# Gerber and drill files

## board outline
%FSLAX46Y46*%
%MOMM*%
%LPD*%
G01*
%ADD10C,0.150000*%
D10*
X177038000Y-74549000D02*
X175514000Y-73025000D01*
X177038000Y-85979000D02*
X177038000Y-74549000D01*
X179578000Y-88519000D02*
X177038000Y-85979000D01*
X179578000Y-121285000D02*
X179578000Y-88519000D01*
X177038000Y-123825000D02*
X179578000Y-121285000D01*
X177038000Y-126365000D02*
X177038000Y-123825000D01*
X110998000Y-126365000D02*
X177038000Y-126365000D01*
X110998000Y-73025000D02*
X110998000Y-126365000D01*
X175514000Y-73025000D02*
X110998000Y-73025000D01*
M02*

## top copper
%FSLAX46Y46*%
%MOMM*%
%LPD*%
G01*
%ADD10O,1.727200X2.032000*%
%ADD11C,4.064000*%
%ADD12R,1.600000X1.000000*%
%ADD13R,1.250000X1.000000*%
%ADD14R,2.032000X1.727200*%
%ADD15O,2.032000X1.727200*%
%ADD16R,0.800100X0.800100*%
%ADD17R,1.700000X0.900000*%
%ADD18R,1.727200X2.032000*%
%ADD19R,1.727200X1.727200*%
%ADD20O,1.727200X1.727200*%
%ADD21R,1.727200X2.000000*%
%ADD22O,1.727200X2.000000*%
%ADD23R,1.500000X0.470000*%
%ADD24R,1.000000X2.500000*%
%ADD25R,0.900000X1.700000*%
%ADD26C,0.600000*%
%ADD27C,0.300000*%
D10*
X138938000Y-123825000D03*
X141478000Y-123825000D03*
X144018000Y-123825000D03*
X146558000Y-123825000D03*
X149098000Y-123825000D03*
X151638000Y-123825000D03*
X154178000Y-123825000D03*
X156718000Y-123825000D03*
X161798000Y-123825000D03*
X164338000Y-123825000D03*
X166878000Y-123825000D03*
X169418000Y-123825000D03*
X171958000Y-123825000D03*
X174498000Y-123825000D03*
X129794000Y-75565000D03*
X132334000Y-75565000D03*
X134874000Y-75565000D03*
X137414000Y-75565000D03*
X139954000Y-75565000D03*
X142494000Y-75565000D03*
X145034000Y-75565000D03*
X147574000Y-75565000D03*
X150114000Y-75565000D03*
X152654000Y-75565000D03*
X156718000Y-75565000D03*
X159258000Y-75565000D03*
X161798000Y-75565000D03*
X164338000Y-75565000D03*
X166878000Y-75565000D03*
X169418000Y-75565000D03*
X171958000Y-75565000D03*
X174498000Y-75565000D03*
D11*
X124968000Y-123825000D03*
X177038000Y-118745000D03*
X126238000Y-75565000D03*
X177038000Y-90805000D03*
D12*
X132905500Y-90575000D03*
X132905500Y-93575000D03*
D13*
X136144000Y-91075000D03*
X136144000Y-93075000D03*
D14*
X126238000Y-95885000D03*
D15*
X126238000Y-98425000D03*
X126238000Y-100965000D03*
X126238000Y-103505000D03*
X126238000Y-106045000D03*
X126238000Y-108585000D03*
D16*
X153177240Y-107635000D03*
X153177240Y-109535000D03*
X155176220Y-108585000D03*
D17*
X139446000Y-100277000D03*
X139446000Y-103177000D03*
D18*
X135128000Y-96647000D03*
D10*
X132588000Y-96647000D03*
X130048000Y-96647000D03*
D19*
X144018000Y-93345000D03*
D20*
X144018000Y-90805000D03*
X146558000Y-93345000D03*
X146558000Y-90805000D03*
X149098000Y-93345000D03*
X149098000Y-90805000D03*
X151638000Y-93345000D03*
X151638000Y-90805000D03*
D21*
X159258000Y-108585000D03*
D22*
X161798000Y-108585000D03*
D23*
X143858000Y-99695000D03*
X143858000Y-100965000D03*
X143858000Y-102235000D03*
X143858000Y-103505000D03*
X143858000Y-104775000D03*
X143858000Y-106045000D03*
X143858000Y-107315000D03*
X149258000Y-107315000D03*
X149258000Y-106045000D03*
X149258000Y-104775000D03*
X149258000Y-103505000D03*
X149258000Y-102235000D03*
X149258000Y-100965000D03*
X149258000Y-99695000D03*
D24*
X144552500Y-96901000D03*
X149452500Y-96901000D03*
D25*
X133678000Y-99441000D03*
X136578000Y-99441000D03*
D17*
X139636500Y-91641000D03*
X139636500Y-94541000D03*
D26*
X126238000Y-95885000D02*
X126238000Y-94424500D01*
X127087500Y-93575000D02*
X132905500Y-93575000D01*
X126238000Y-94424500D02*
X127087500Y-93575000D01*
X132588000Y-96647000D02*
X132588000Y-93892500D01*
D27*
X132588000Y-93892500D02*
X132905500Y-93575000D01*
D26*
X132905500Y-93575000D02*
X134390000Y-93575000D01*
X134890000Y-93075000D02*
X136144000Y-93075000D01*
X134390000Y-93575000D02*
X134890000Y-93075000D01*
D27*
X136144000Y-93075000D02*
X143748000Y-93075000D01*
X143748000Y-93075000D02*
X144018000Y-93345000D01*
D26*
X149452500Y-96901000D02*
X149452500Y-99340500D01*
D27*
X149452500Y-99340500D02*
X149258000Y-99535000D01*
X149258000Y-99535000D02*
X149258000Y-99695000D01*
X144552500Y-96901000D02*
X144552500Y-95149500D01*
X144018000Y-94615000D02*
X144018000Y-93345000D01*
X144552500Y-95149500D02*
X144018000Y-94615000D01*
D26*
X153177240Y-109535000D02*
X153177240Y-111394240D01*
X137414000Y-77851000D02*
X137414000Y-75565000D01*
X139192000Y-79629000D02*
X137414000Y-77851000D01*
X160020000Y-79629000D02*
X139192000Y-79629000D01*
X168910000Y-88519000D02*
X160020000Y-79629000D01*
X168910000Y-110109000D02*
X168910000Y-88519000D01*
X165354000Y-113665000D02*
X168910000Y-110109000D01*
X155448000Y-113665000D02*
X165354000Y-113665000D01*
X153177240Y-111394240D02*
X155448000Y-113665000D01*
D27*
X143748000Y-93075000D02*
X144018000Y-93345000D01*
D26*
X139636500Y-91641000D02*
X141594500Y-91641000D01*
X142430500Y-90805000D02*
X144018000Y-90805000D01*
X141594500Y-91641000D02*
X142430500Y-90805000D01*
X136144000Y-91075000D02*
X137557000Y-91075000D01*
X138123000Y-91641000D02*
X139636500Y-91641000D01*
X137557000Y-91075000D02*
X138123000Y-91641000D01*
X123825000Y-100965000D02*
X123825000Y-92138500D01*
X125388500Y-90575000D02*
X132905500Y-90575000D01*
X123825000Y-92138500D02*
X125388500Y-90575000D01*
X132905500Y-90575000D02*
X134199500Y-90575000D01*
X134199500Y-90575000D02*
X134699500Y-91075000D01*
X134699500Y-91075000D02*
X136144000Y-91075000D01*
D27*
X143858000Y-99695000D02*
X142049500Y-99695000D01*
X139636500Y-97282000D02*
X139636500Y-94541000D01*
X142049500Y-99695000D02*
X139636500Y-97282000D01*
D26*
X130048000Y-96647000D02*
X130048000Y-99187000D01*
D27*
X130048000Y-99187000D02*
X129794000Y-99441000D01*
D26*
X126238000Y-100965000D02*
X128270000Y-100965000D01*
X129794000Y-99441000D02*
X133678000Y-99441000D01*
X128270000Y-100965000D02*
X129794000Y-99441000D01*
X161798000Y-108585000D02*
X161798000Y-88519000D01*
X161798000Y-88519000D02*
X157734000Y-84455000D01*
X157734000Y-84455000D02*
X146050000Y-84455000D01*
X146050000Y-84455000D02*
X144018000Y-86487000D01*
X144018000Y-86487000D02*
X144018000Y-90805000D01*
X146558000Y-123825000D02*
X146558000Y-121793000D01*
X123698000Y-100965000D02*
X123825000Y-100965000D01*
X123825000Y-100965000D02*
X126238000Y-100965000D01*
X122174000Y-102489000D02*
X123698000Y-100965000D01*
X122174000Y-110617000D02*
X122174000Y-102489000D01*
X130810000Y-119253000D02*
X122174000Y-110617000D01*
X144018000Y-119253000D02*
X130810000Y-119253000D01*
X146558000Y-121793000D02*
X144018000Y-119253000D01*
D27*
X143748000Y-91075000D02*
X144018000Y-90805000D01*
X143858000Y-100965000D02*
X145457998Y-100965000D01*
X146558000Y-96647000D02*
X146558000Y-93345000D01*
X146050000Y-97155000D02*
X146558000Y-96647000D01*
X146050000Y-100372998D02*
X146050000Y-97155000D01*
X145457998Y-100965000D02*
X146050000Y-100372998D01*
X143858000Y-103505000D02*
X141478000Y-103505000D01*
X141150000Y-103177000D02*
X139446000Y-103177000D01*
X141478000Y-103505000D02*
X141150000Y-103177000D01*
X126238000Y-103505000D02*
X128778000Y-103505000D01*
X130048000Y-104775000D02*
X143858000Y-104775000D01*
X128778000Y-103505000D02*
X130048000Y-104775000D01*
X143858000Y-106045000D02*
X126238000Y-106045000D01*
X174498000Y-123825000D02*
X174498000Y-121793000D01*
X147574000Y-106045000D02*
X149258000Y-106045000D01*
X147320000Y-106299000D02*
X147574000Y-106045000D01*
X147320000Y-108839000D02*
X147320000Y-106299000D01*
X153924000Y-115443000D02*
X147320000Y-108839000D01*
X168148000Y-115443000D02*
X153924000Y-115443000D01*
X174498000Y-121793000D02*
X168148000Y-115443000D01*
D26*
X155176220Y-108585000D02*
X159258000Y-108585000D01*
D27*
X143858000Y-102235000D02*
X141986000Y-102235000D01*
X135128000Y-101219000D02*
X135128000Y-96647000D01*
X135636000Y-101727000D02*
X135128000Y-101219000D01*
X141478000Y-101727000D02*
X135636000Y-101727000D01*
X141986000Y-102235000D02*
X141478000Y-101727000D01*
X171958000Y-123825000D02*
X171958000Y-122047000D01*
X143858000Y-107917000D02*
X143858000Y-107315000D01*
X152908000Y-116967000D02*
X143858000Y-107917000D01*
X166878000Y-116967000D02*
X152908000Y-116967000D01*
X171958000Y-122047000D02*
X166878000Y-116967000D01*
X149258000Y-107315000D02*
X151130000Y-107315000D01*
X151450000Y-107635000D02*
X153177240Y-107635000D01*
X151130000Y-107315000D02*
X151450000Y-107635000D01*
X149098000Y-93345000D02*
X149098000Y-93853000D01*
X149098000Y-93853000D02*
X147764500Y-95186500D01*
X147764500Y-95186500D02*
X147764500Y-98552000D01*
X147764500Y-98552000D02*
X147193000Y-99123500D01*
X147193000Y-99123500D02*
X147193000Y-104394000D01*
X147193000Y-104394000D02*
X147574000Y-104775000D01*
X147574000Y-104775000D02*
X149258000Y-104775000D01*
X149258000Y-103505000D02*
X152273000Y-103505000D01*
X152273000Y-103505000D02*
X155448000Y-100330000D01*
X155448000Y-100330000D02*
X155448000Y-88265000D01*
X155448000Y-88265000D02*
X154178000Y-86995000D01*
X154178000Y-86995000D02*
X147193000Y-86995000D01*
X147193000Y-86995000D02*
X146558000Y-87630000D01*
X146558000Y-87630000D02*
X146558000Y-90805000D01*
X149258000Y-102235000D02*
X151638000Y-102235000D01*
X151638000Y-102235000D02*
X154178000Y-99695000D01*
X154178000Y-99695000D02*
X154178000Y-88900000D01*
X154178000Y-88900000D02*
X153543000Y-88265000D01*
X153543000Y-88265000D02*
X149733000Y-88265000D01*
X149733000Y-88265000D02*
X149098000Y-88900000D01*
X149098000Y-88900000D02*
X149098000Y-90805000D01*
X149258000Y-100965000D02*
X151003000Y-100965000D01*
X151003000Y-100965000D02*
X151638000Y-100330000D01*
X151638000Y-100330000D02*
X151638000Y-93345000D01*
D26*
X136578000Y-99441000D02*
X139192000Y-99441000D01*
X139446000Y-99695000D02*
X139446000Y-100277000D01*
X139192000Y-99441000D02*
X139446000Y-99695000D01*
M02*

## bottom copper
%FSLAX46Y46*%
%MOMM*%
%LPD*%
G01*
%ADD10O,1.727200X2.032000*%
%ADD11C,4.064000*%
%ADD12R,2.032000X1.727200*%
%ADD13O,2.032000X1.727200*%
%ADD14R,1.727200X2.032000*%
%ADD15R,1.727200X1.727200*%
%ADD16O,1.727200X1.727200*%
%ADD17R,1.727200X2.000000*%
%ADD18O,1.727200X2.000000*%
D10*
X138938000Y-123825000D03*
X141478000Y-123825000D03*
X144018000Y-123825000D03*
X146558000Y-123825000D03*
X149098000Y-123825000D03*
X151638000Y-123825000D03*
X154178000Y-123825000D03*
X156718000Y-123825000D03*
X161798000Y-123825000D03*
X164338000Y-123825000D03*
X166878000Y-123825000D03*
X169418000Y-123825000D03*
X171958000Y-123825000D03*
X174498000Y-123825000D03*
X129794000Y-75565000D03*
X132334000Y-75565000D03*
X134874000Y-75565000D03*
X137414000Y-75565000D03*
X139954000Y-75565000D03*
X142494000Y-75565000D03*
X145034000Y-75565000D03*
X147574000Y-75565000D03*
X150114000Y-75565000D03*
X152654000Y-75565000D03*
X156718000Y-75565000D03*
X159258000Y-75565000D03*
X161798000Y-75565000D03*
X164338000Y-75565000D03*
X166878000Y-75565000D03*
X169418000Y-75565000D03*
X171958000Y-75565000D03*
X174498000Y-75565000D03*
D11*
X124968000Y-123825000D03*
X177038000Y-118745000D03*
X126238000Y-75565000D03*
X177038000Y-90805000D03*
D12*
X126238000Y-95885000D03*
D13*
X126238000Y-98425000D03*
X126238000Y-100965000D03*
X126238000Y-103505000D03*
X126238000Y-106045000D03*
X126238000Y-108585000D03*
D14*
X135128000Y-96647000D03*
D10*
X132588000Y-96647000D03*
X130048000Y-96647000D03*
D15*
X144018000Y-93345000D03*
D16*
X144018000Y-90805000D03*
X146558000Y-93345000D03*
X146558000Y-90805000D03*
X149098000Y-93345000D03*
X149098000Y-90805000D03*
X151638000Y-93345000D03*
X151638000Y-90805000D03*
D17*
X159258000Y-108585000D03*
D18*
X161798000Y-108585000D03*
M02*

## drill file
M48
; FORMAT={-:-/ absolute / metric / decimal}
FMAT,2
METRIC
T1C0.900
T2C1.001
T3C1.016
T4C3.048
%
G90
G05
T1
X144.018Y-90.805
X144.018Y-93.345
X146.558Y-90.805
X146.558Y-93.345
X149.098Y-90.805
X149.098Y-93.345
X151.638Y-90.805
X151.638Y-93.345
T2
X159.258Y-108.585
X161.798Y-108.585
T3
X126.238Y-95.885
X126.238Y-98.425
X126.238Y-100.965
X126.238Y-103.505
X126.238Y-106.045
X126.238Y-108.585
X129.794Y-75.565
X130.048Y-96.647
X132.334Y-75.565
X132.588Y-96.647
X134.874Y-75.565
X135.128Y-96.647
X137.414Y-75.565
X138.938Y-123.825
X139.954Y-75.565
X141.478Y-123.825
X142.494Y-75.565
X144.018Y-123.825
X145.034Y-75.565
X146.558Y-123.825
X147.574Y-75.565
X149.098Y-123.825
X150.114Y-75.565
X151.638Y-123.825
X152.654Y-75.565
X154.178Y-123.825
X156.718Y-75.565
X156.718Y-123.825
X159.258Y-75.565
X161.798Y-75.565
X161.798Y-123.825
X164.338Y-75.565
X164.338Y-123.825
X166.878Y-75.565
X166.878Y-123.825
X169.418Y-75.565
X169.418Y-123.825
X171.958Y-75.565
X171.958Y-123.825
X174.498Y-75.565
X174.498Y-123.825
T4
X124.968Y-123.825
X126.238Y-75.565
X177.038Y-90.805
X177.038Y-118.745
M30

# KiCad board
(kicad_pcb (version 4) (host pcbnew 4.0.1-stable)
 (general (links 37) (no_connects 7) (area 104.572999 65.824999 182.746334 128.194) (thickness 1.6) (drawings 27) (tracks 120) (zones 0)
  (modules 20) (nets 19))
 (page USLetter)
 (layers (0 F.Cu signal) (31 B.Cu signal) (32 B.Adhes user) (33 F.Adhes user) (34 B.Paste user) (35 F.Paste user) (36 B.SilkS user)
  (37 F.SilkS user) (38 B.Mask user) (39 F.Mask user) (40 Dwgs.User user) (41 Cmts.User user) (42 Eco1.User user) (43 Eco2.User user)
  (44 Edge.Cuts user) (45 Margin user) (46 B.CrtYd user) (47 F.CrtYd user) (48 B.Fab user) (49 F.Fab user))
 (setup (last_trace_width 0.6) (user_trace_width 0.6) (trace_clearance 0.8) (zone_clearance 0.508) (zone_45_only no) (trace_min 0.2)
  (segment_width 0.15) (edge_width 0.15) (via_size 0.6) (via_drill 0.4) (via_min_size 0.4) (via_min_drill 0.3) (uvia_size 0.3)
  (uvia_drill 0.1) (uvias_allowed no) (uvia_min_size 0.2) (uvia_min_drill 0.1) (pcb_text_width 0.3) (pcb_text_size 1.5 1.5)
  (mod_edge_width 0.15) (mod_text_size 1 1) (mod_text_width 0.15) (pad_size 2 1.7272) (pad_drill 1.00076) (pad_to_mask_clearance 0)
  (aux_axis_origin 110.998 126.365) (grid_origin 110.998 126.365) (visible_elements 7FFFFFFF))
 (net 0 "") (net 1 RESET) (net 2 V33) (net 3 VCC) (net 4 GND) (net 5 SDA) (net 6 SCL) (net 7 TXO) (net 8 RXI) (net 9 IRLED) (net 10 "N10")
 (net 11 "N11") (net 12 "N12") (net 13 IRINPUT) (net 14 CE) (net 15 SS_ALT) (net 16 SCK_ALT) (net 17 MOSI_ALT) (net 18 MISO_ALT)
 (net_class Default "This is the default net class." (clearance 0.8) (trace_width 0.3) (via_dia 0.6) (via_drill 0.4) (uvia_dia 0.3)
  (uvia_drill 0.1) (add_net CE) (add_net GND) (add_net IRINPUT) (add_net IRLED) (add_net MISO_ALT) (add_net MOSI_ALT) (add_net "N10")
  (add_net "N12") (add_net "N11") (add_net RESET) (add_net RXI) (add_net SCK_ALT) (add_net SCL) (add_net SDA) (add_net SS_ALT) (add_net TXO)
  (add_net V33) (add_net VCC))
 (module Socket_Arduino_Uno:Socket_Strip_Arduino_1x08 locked (layer F.Cu) (at 138.938 123.825)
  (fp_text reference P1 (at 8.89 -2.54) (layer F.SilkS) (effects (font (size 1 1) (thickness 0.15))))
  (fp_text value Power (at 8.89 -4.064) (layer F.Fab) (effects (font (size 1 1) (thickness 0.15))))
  (pad 1 thru_hole oval (at 0 0) (size 1.7272 2.032) (drill 1.016) (layers *.Cu *.Mask F.SilkS))
  (pad 2 thru_hole oval (at 2.54 0) (size 1.7272 2.032) (drill 1.016) (layers *.Cu *.Mask F.SilkS))
  (pad 3 thru_hole oval (at 5.08 0) (size 1.7272 2.032) (drill 1.016) (layers *.Cu *.Mask F.SilkS) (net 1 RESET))
  (pad 4 thru_hole oval (at 7.62 0) (size 1.7272 2.032) (drill 1.016) (layers *.Cu *.Mask F.SilkS) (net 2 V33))
  (pad 5 thru_hole oval (at 10.16 0) (size 1.7272 2.032) (drill 1.016) (layers *.Cu *.Mask F.SilkS) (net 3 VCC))
  (pad 6 thru_hole oval (at 12.7 0) (size 1.7272 2.032) (drill 1.016) (layers *.Cu *.Mask F.SilkS) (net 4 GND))
  (pad 7 thru_hole oval (at 15.24 0) (size 1.7272 2.032) (drill 1.016) (layers *.Cu *.Mask F.SilkS) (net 4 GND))
  (pad 8 thru_hole oval (at 17.78 0) (size 1.7272 2.032) (drill 1.016) (layers *.Cu *.Mask F.SilkS)))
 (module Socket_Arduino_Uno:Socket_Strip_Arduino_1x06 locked (layer F.Cu) (at 161.798 123.825)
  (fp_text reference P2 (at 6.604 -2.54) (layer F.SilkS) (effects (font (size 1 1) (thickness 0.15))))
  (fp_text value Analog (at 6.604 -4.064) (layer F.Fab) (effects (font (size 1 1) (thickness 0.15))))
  (pad 1 thru_hole oval (at 0 0) (size 1.7272 2.032) (drill 1.016) (layers *.Cu *.Mask F.SilkS))
  (pad 2 thru_hole oval (at 2.54 0) (size 1.7272 2.032) (drill 1.016) (layers *.Cu *.Mask F.SilkS))
  (pad 3 thru_hole oval (at 5.08 0) (size 1.7272 2.032) (drill 1.016) (layers *.Cu *.Mask F.SilkS))
  (pad 4 thru_hole oval (at 7.62 0) (size 1.7272 2.032) (drill 1.016) (layers *.Cu *.Mask F.SilkS))
  (pad 5 thru_hole oval (at 10.16 0) (size 1.7272 2.032) (drill 1.016) (layers *.Cu *.Mask F.SilkS) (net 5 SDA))
  (pad 6 thru_hole oval (at 12.7 0) (size 1.7272 2.032) (drill 1.016) (layers *.Cu *.Mask F.SilkS) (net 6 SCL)))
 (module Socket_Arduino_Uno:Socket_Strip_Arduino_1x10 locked (layer F.Cu) (at 129.794 75.565)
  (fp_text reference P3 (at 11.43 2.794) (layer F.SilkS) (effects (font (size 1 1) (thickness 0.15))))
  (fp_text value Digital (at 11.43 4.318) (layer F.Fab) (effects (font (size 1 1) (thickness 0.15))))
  (pad 1 thru_hole oval (at 0 0) (size 1.7272 2.032) (drill 1.016) (layers *.Cu *.Mask F.SilkS) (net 6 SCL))
  (pad 2 thru_hole oval (at 2.54 0) (size 1.7272 2.032) (drill 1.016) (layers *.Cu *.Mask F.SilkS) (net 5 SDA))
  (pad 3 thru_hole oval (at 5.08 0) (size 1.7272 2.032) (drill 1.016) (layers *.Cu *.Mask F.SilkS))
  (pad 4 thru_hole oval (at 7.62 0) (size 1.7272 2.032) (drill 1.016) (layers *.Cu *.Mask F.SilkS) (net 4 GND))
  (pad 5 thru_hole oval (at 10.16 0) (size 1.7272 2.032) (drill 1.016) (layers *.Cu *.Mask F.SilkS))
  (pad 6 thru_hole oval (at 12.7 0) (size 1.7272 2.032) (drill 1.016) (layers *.Cu *.Mask F.SilkS))
  (pad 7 thru_hole oval (at 15.24 0) (size 1.7272 2.032) (drill 1.016) (layers *.Cu *.Mask F.SilkS))
  (pad 8 thru_hole oval (at 17.78 0) (size 1.7272 2.032) (drill 1.016) (layers *.Cu *.Mask F.SilkS))
  (pad 9 thru_hole oval (at 20.32 0) (size 1.7272 2.032) (drill 1.016) (layers *.Cu *.Mask F.SilkS))
  (pad 10 thru_hole oval (at 22.86 0) (size 1.7272 2.032) (drill 1.016) (layers *.Cu *.Mask F.SilkS)))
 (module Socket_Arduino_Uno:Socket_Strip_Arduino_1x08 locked (layer F.Cu) (at 156.718 75.565)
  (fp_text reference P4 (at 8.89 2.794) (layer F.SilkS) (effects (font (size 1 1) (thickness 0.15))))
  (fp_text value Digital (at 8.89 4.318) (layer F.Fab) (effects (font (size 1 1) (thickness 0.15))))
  (pad 1 thru_hole oval (at 0 0) (size 1.7272 2.032) (drill 1.016) (layers *.Cu *.Mask F.SilkS))
  (pad 2 thru_hole oval (at 2.54 0) (size 1.7272 2.032) (drill 1.016) (layers *.Cu *.Mask F.SilkS))
  (pad 3 thru_hole oval (at 5.08 0) (size 1.7272 2.032) (drill 1.016) (layers *.Cu *.Mask F.SilkS))
  (pad 4 thru_hole oval (at 7.62 0) (size 1.7272 2.032) (drill 1.016) (layers *.Cu *.Mask F.SilkS))
  (pad 5 thru_hole oval (at 10.16 0) (size 1.7272 2.032) (drill 1.016) (layers *.Cu *.Mask F.SilkS))
  (pad 6 thru_hole oval (at 12.7 0) (size 1.7272 2.032) (drill 1.016) (layers *.Cu *.Mask F.SilkS))
  (pad 7 thru_hole oval (at 15.24 0) (size 1.7272 2.032) (drill 1.016) (layers *.Cu *.Mask F.SilkS))
  (pad 8 thru_hole oval (at 17.78 0) (size 1.7272 2.032) (drill 1.016) (layers *.Cu *.Mask F.SilkS)))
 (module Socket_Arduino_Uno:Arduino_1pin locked (layer F.Cu) (at 124.968 123.825)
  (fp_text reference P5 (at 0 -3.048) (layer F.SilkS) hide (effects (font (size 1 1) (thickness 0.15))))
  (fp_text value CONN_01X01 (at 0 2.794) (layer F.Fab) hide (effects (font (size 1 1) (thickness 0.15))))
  (pad 1 thru_hole circle (at 0 0) (size 4.064 4.064) (drill 3.048) (layers *.Cu *.Mask F.SilkS)))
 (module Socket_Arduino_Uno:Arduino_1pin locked (layer F.Cu) (at 177.038 118.745)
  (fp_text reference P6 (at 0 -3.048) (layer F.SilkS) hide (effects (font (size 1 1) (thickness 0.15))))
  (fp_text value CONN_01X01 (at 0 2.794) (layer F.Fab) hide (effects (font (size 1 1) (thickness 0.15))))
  (pad 1 thru_hole circle (at 0 0) (size 4.064 4.064) (drill 3.048) (layers *.Cu *.Mask F.SilkS)))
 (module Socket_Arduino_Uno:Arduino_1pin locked (layer F.Cu) (at 126.238 75.565)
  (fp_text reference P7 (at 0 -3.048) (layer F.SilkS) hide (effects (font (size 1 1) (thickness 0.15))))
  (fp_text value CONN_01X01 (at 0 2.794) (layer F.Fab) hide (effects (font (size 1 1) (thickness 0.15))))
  (pad 1 thru_hole circle (at 0 0) (size 4.064 4.064) (drill 3.048) (layers *.Cu *.Mask F.SilkS)))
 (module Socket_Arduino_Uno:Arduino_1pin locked (layer F.Cu) (at 177.038 90.805)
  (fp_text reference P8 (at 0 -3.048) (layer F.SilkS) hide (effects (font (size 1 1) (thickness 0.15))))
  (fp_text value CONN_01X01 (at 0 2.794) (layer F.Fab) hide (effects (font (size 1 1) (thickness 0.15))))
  (pad 1 thru_hole circle (at 0 0) (size 4.064 4.064) (drill 3.048) (layers *.Cu *.Mask F.SilkS)))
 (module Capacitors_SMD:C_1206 (layer F.Cu) (at 132.9055 92.075 270)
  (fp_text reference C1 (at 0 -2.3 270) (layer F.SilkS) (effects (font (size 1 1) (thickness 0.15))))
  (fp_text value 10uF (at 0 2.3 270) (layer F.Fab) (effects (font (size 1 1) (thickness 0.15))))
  (pad 1 smd rect (at -1.5 0 270) (size 1 1.6) (layers F.Cu F.Paste F.Mask) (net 2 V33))
  (pad 2 smd rect (at 1.5 0 270) (size 1 1.6) (layers F.Cu F.Paste F.Mask) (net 4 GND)))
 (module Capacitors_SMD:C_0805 (layer F.Cu) (at 136.144 92.075 270)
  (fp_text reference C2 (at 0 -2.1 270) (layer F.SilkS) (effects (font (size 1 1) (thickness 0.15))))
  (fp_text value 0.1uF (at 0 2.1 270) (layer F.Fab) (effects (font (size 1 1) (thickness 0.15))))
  (pad 1 smd rect (at -1 0 270) (size 1 1.25) (layers F.Cu F.Paste F.Mask) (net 2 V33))
  (pad 2 smd rect (at 1 0 270) (size 1 1.25) (layers F.Cu F.Paste F.Mask) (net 4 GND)))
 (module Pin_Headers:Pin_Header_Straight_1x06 (layer F.Cu) (at 126.238 95.885)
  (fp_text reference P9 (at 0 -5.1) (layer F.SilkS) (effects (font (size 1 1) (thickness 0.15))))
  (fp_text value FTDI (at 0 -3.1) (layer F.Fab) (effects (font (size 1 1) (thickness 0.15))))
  (pad 1 thru_hole rect (at 0 0) (size 2.032 1.7272) (drill 1.016) (layers *.Cu *.Mask F.SilkS) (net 4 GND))
  (pad 2 thru_hole oval (at 0 2.54) (size 2.032 1.7272) (drill 1.016) (layers *.Cu *.Mask F.SilkS))
  (pad 3 thru_hole oval (at 0 5.08) (size 2.032 1.7272) (drill 1.016) (layers *.Cu *.Mask F.SilkS) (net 2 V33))
  (pad 4 thru_hole oval (at 0 7.62) (size 2.032 1.7272) (drill 1.016) (layers *.Cu *.Mask F.SilkS) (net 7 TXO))
  (pad 5 thru_hole oval (at 0 10.16) (size 2.032 1.7272) (drill 1.016) (layers *.Cu *.Mask F.SilkS) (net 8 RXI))
  (pad 6 thru_hole oval (at 0 12.7) (size 2.032 1.7272) (drill 1.016) (layers *.Cu *.Mask F.SilkS)))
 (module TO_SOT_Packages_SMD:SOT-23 (layer F.Cu) (at 154.178 108.585 270)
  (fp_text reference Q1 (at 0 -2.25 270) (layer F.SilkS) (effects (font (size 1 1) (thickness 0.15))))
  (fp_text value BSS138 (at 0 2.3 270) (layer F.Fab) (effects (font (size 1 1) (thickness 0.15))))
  (pad 1 smd rect (at -0.95 1.00076 270) (size 0.8001 0.8001) (layers F.Cu F.Paste F.Mask) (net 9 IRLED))
  (pad 2 smd rect (at 0.95 1.00076 270) (size 0.8001 0.8001) (layers F.Cu F.Paste F.Mask) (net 4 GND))
  (pad 3 smd rect (at 0 -0.99822 270) (size 0.8001 0.8001) (layers F.Cu F.Paste F.Mask) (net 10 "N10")))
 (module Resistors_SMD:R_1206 (layer F.Cu) (at 139.446 101.727 270)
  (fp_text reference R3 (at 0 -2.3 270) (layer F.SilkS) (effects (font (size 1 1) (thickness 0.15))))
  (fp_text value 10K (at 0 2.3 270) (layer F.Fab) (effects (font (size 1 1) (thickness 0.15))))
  (pad 1 smd rect (at -1.45 0 270) (size 0.9 1.7) (layers F.Cu F.Paste F.Mask) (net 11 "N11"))
  (pad 2 smd rect (at 1.45 0 270) (size 0.9 1.7) (layers F.Cu F.Paste F.Mask) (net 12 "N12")))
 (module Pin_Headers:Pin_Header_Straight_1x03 (layer F.Cu) (at 135.128 96.647 270)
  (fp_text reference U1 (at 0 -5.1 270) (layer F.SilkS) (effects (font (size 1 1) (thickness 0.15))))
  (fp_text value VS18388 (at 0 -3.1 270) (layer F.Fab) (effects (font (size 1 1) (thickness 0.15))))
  (pad 1 thru_hole rect (at 0 0 270) (size 2.032 1.7272) (drill 1.016) (layers *.Cu *.Mask F.SilkS) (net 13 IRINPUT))
  (pad 2 thru_hole oval (at 0 2.54 270) (size 2.032 1.7272) (drill 1.016) (layers *.Cu *.Mask F.SilkS) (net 4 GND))
  (pad 3 thru_hole oval (at 0 5.08 270) (size 2.032 1.7272) (drill 1.016) (layers *.Cu *.Mask F.SilkS) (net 2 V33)))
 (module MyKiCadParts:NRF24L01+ (layer F.Cu) (at 144.018 93.345 90)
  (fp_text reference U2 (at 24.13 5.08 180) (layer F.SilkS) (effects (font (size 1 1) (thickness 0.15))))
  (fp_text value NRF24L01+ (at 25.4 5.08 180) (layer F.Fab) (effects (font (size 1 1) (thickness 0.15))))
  (pad 1 thru_hole rect (at 0 0 90) (size 1.7272 1.7272) (drill 0.9) (layers *.Cu *.Mask F.SilkS) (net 4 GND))
  (pad 2 thru_hole oval (at 2.54 0 90) (size 1.7272 1.7272) (drill 0.9) (layers *.Cu *.Mask F.SilkS) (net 2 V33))
  (pad 3 thru_hole oval (at 0 2.54 90) (size 1.7272 1.7272) (drill 0.9) (layers *.Cu *.Mask F.SilkS) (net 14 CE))
  (pad 4 thru_hole oval (at 2.54 2.54 90) (size 1.7272 1.7272) (drill 0.9) (layers *.Cu *.Mask F.SilkS) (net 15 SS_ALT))
  (pad 5 thru_hole oval (at 0 5.08 90) (size 1.7272 1.7272) (drill 0.9) (layers *.Cu *.Mask F.SilkS) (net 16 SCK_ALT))
  (pad 6 thru_hole oval (at 2.54 5.08 90) (size 1.7272 1.7272) (drill 0.9) (layers *.Cu *.Mask F.SilkS) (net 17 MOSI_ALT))
  (pad 7 thru_hole oval (at 0 7.62 90) (size 1.7272 1.7272) (drill 0.9) (layers *.Cu *.Mask F.SilkS) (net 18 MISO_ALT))
  (pad 8 thru_hole oval (at 2.54 7.62 90) (size 1.7272 1.7272) (drill 0.9) (layers *.Cu *.Mask F.SilkS)))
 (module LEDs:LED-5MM (layer F.Cu) (at 159.258 108.585)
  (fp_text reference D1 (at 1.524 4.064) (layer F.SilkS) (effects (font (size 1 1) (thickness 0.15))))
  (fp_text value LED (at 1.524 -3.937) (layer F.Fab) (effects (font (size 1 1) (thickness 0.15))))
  (pad 1 thru_hole rect (at 0 0 90) (size 2 1.7272) (drill 1.00076) (layers *.Cu *.Mask F.SilkS) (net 10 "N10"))
  (pad 2 thru_hole oval (at 2.54 0) (size 1.7272 2) (drill 1.00076) (layers *.Cu *.Mask F.SilkS) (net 2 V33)))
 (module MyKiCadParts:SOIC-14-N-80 (layer F.Cu) (at 146.558 103.505)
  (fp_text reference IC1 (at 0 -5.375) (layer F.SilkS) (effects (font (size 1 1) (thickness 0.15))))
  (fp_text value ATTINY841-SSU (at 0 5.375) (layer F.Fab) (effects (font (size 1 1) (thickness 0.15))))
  (pad 1 smd rect (at -2.7 -3.81) (size 1.5 0.47) (layers F.Cu F.Paste F.Mask) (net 2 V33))
  (pad 2 smd rect (at -2.7 -2.54) (size 1.5 0.47) (layers F.Cu F.Paste F.Mask) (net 14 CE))
  (pad 3 smd rect (at -2.7 -1.27) (size 1.5 0.47) (layers F.Cu F.Paste F.Mask) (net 13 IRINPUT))
  (pad 4 smd rect (at -2.7 0) (size 1.5 0.47) (layers F.Cu F.Paste F.Mask) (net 12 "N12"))
  (pad 5 smd rect (at -2.7 1.27) (size 1.5 0.47) (layers F.Cu F.Paste F.Mask) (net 7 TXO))
  (pad 6 smd rect (at -2.7 2.54) (size 1.5 0.47) (layers F.Cu F.Paste F.Mask) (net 8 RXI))
  (pad 7 smd rect (at -2.7 3.81) (size 1.5 0.47) (layers F.Cu F.Paste F.Mask) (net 5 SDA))
  (pad 8 smd rect (at 2.7 3.81) (size 1.5 0.47) (layers F.Cu F.Paste F.Mask) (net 9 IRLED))
  (pad 9 smd rect (at 2.7 2.54) (size 1.5 0.47) (layers F.Cu F.Paste F.Mask) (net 6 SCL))
  (pad 10 smd rect (at 2.7 1.27) (size 1.5 0.47) (layers F.Cu F.Paste F.Mask) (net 16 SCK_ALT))
  (pad 11 smd rect (at 2.7 0) (size 1.5 0.47) (layers F.Cu F.Paste F.Mask) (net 15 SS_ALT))
  (pad 12 smd rect (at 2.7 -1.27) (size 1.5 0.47) (layers F.Cu F.Paste F.Mask) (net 17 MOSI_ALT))
  (pad 13 smd rect (at 2.7 -2.54) (size 1.5 0.47) (layers F.Cu F.Paste F.Mask) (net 18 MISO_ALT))
  (pad 14 smd rect (at 2.7 -3.81) (size 1.5 0.47) (layers F.Cu F.Paste F.Mask) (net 4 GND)))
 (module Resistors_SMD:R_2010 (layer F.Cu) (at 147.0025 96.901)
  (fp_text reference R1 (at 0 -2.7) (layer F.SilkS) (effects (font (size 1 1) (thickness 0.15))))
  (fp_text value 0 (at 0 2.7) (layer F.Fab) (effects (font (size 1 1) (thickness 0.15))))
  (pad 1 smd rect (at -2.45 0) (size 1 2.5) (layers F.Cu F.Paste F.Mask) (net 4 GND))
  (pad 2 smd rect (at 2.45 0) (size 1 2.5) (layers F.Cu F.Paste F.Mask) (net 4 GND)))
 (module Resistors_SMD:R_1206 (layer F.Cu) (at 135.128 99.441)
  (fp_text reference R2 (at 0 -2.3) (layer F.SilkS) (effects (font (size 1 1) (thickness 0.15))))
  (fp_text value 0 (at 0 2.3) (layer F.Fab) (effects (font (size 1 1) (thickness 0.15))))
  (pad 1 smd rect (at -1.45 0) (size 0.9 1.7) (layers F.Cu F.Paste F.Mask) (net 2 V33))
  (pad 2 smd rect (at 1.45 0) (size 0.9 1.7) (layers F.Cu F.Paste F.Mask) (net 11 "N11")))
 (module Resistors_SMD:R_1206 (layer F.Cu) (at 139.6365 93.091 270)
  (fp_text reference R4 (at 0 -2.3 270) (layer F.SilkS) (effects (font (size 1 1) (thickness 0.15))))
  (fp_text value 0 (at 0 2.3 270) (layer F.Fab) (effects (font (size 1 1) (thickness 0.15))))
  (pad 1 smd rect (at -1.45 0 270) (size 0.9 1.7) (layers F.Cu F.Paste F.Mask) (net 2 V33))
  (pad 2 smd rect (at 1.45 0 270) (size 0.9 1.7) (layers F.Cu F.Paste F.Mask) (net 2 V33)))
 (gr_line (start 177.038 74.549) (end 175.514 73.025) (angle 90) (layer Edge.Cuts) (width 0.15))
 (gr_line (start 177.038 85.979) (end 177.038 74.549) (angle 90) (layer Edge.Cuts) (width 0.15))
 (gr_line (start 179.578 88.519) (end 177.038 85.979) (angle 90) (layer Edge.Cuts) (width 0.15))
 (gr_line (start 179.578 121.285) (end 179.578 88.519) (angle 90) (layer Edge.Cuts) (width 0.15))
 (gr_line (start 177.038 123.825) (end 179.578 121.285) (angle 90) (layer Edge.Cuts) (width 0.15))
 (gr_line (start 177.038 126.365) (end 177.038 123.825) (angle 90) (layer Edge.Cuts) (width 0.15))
 (gr_line (start 110.998 126.365) (end 177.038 126.365) (angle 90) (layer Edge.Cuts) (width 0.15))
 (gr_line (start 110.998 73.025) (end 110.998 126.365) (angle 90) (layer Edge.Cuts) (width 0.15))
 (gr_line (start 175.514 73.025) (end 110.998 73.025) (angle 90) (layer Edge.Cuts) (width 0.15))
 (segment (start 126.238 95.885) (end 126.238 94.4245) (width 0.6) (layer F.Cu) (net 4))
 (segment (start 127.0875 93.575) (end 132.9055 93.575) (width 0.6) (layer F.Cu) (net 4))
 (segment (start 126.238 94.4245) (end 127.0875 93.575) (width 0.6) (layer F.Cu) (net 4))
 (segment (start 132.588 96.647) (end 132.588 93.8925) (width 0.6) (layer F.Cu) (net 4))
 (segment (start 132.588 93.8925) (end 132.9055 93.575) (width 0.3) (layer F.Cu) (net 4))
 (segment (start 132.9055 93.575) (end 134.39 93.575) (width 0.6) (layer F.Cu) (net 4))
 (segment (start 134.89 93.075) (end 136.144 93.075) (width 0.6) (layer F.Cu) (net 4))
 (segment (start 134.39 93.575) (end 134.89 93.075) (width 0.6) (layer F.Cu) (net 4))
 (segment (start 136.144 93.075) (end 143.748 93.075) (width 0.3) (layer F.Cu) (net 4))
 (segment (start 143.748 93.075) (end 144.018 93.345) (width 0.3) (layer F.Cu) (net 4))
 (segment (start 149.4525 96.901) (end 149.4525 99.3405) (width 0.6) (layer F.Cu) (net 4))
 (segment (start 149.4525 99.3405) (end 149.258 99.535) (width 0.3) (layer F.Cu) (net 4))
 (segment (start 149.258 99.535) (end 149.258 99.695) (width 0.3) (layer F.Cu) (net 4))
 (segment (start 144.5525 96.901) (end 144.5525 95.1495) (width 0.3) (layer F.Cu) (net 4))
 (segment (start 144.018 94.615) (end 144.018 93.345) (width 0.3) (layer F.Cu) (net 4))
 (segment (start 144.5525 95.1495) (end 144.018 94.615) (width 0.3) (layer F.Cu) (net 4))
 (segment (start 153.17724 109.535) (end 153.17724 111.39424) (width 0.6) (layer F.Cu) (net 4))
 (segment (start 137.414 77.851) (end 137.414 75.565) (width 0.6) (layer F.Cu) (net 4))
 (segment (start 139.192 79.629) (end 137.414 77.851) (width 0.6) (layer F.Cu) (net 4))
 (segment (start 160.02 79.629) (end 139.192 79.629) (width 0.6) (layer F.Cu) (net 4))
 (segment (start 168.91 88.519) (end 160.02 79.629) (width 0.6) (layer F.Cu) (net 4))
 (segment (start 168.91 110.109) (end 168.91 88.519) (width 0.6) (layer F.Cu) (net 4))
 (segment (start 165.354 113.665) (end 168.91 110.109) (width 0.6) (layer F.Cu) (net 4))
 (segment (start 155.448 113.665) (end 165.354 113.665) (width 0.6) (layer F.Cu) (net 4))
 (segment (start 153.17724 111.39424) (end 155.448 113.665) (width 0.6) (layer F.Cu) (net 4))
 (segment (start 143.748 93.075) (end 144.018 93.345) (width 0.3) (layer F.Cu) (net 4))
 (segment (start 139.6365 91.641) (end 141.5945 91.641) (width 0.6) (layer F.Cu) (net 2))
 (segment (start 142.4305 90.805) (end 144.018 90.805) (width 0.6) (layer F.Cu) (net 2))
 (segment (start 141.5945 91.641) (end 142.4305 90.805) (width 0.6) (layer F.Cu) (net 2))
 (segment (start 136.144 91.075) (end 137.557 91.075) (width 0.6) (layer F.Cu) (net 2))
 (segment (start 138.123 91.641) (end 139.6365 91.641) (width 0.6) (layer F.Cu) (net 2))
 (segment (start 137.557 91.075) (end 138.123 91.641) (width 0.6) (layer F.Cu) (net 2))
 (segment (start 123.825 100.965) (end 123.825 92.1385) (width 0.6) (layer F.Cu) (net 2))
 (segment (start 125.3885 90.575) (end 132.9055 90.575) (width 0.6) (layer F.Cu) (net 2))
 (segment (start 123.825 92.1385) (end 125.3885 90.575) (width 0.6) (layer F.Cu) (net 2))
 (segment (start 132.9055 90.575) (end 134.1995 90.575) (width 0.6) (layer F.Cu) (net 2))
 (segment (start 134.1995 90.575) (end 134.6995 91.075) (width 0.6) (layer F.Cu) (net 2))
 (segment (start 134.6995 91.075) (end 136.144 91.075) (width 0.6) (layer F.Cu) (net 2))
 (segment (start 143.858 99.695) (end 142.0495 99.695) (width 0.3) (layer F.Cu) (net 2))
 (segment (start 139.6365 97.282) (end 139.6365 94.541) (width 0.3) (layer F.Cu) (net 2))
 (segment (start 142.0495 99.695) (end 139.6365 97.282) (width 0.3) (layer F.Cu) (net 2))
 (segment (start 130.048 96.647) (end 130.048 99.187) (width 0.6) (layer F.Cu) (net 2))
 (segment (start 130.048 99.187) (end 129.794 99.441) (width 0.3) (layer F.Cu) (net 2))
 (segment (start 126.238 100.965) (end 128.27 100.965) (width 0.6) (layer F.Cu) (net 2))
 (segment (start 129.794 99.441) (end 133.678 99.441) (width 0.6) (layer F.Cu) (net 2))
 (segment (start 128.27 100.965) (end 129.794 99.441) (width 0.6) (layer F.Cu) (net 2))
 (segment (start 161.798 108.585) (end 161.798 88.519) (width 0.6) (layer F.Cu) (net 2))
 (segment (start 161.798 88.519) (end 157.734 84.455) (width 0.6) (layer F.Cu) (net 2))
 (segment (start 157.734 84.455) (end 146.05 84.455) (width 0.6) (layer F.Cu) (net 2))
 (segment (start 146.05 84.455) (end 144.018 86.487) (width 0.6) (layer F.Cu) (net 2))
 (segment (start 144.018 86.487) (end 144.018 90.805) (width 0.6) (layer F.Cu) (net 2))
 (segment (start 146.558 123.825) (end 146.558 121.793) (width 0.6) (layer F.Cu) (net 2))
 (segment (start 123.698 100.965) (end 123.825 100.965) (width 0.6) (layer F.Cu) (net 2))
 (segment (start 123.825 100.965) (end 126.238 100.965) (width 0.6) (layer F.Cu) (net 2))
 (segment (start 122.174 102.489) (end 123.698 100.965) (width 0.6) (layer F.Cu) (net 2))
 (segment (start 122.174 110.617) (end 122.174 102.489) (width 0.6) (layer F.Cu) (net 2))
 (segment (start 130.81 119.253) (end 122.174 110.617) (width 0.6) (layer F.Cu) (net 2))
 (segment (start 144.018 119.253) (end 130.81 119.253) (width 0.6) (layer F.Cu) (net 2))
 (segment (start 146.558 121.793) (end 144.018 119.253) (width 0.6) (layer F.Cu) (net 2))
 (segment (start 143.748 91.075) (end 144.018 90.805) (width 0.3) (layer F.Cu) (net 2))
 (segment (start 143.858 100.965) (end 145.457998 100.965) (width 0.3) (layer F.Cu) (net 14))
 (segment (start 146.558 96.647) (end 146.558 93.345) (width 0.3) (layer F.Cu) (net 14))
 (segment (start 146.05 97.155) (end 146.558 96.647) (width 0.3) (layer F.Cu) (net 14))
 (segment (start 146.05 100.372998) (end 146.05 97.155) (width 0.3) (layer F.Cu) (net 14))
 (segment (start 145.457998 100.965) (end 146.05 100.372998) (width 0.3) (layer F.Cu) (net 14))
 (segment (start 143.858 103.505) (end 141.478 103.505) (width 0.3) (layer F.Cu) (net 12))
 (segment (start 141.15 103.177) (end 139.446 103.177) (width 0.3) (layer F.Cu) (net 12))
 (segment (start 141.478 103.505) (end 141.15 103.177) (width 0.3) (layer F.Cu) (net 12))
 (segment (start 126.238 103.505) (end 128.778 103.505) (width 0.3) (layer F.Cu) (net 7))
 (segment (start 130.048 104.775) (end 143.858 104.775) (width 0.3) (layer F.Cu) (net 7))
 (segment (start 128.778 103.505) (end 130.048 104.775) (width 0.3) (layer F.Cu) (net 7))
 (segment (start 143.858 106.045) (end 126.238 106.045) (width 0.3) (layer F.Cu) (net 8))
 (segment (start 174.498 123.825) (end 174.498 121.793) (width 0.3) (layer F.Cu) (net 6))
 (segment (start 147.574 106.045) (end 149.258 106.045) (width 0.3) (layer F.Cu) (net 6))
 (segment (start 147.32 106.299) (end 147.574 106.045) (width 0.3) (layer F.Cu) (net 6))
 (segment (start 147.32 108.839) (end 147.32 106.299) (width 0.3) (layer F.Cu) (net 6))
 (segment (start 153.924 115.443) (end 147.32 108.839) (width 0.3) (layer F.Cu) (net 6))
 (segment (start 168.148 115.443) (end 153.924 115.443) (width 0.3) (layer F.Cu) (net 6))
 (segment (start 174.498 121.793) (end 168.148 115.443) (width 0.3) (layer F.Cu) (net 6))
 (segment (start 155.17622 108.585) (end 159.258 108.585) (width 0.6) (layer F.Cu) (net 10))
 (segment (start 143.858 102.235) (end 141.986 102.235) (width 0.3) (layer F.Cu) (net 13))
 (segment (start 135.128 101.219) (end 135.128 96.647) (width 0.3) (layer F.Cu) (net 13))
 (segment (start 135.636 101.727) (end 135.128 101.219) (width 0.3) (layer F.Cu) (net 13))
 (segment (start 141.478 101.727) (end 135.636 101.727) (width 0.3) (layer F.Cu) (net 13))
 (segment (start 141.986 102.235) (end 141.478 101.727) (width 0.3) (layer F.Cu) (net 13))
 (segment (start 171.958 123.825) (end 171.958 122.047) (width 0.3) (layer F.Cu) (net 5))
 (segment (start 143.858 107.917) (end 143.858 107.315) (width 0.3) (layer F.Cu) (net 5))
 (segment (start 152.908 116.967) (end 143.858 107.917) (width 0.3) (layer F.Cu) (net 5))
 (segment (start 166.878 116.967) (end 152.908 116.967) (width 0.3) (layer F.Cu) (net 5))
 (segment (start 171.958 122.047) (end 166.878 116.967) (width 0.3) (layer F.Cu) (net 5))
 (segment (start 149.258 107.315) (end 151.13 107.315) (width 0.3) (layer F.Cu) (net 9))
 (segment (start 151.45 107.635) (end 153.17724 107.635) (width 0.3) (layer F.Cu) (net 9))
 (segment (start 151.13 107.315) (end 151.45 107.635) (width 0.3) (layer F.Cu) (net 9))
 (segment (start 149.098 93.345) (end 149.098 93.853) (width 0.3) (layer F.Cu) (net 16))
 (segment (start 149.098 93.853) (end 147.7645 95.1865) (width 0.3) (layer F.Cu) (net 16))
 (segment (start 147.7645 95.1865) (end 147.7645 98.552) (width 0.3) (layer F.Cu) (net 16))
 (segment (start 147.7645 98.552) (end 147.193 99.1235) (width 0.3) (layer F.Cu) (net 16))
 (segment (start 147.193 99.1235) (end 147.193 104.394) (width 0.3) (layer F.Cu) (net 16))
 (segment (start 147.193 104.394) (end 147.574 104.775) (width 0.3) (layer F.Cu) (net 16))
 (segment (start 147.574 104.775) (end 149.258 104.775) (width 0.3) (layer F.Cu) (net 16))
 (segment (start 149.258 103.505) (end 152.273 103.505) (width 0.3) (layer F.Cu) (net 15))
 (segment (start 152.273 103.505) (end 155.448 100.33) (width 0.3) (layer F.Cu) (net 15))
 (segment (start 155.448 100.33) (end 155.448 88.265) (width 0.3) (layer F.Cu) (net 15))
 (segment (start 155.448 88.265) (end 154.178 86.995) (width 0.3) (layer F.Cu) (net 15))
 (segment (start 154.178 86.995) (end 147.193 86.995) (width 0.3) (layer F.Cu) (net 15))
 (segment (start 147.193 86.995) (end 146.558 87.63) (width 0.3) (layer F.Cu) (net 15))
 (segment (start 146.558 87.63) (end 146.558 90.805) (width 0.3) (layer F.Cu) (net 15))
 (segment (start 149.258 102.235) (end 151.638 102.235) (width 0.3) (layer F.Cu) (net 17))
 (segment (start 151.638 102.235) (end 154.178 99.695) (width 0.3) (layer F.Cu) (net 17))
 (segment (start 154.178 99.695) (end 154.178 88.9) (width 0.3) (layer F.Cu) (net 17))
 (segment (start 154.178 88.9) (end 153.543 88.265) (width 0.3) (layer F.Cu) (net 17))
 (segment (start 153.543 88.265) (end 149.733 88.265) (width 0.3) (layer F.Cu) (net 17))
 (segment (start 149.733 88.265) (end 149.098 88.9) (width 0.3) (layer F.Cu) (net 17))
 (segment (start 149.098 88.9) (end 149.098 90.805) (width 0.3) (layer F.Cu) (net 17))
 (segment (start 149.258 100.965) (end 151.003 100.965) (width 0.3) (layer F.Cu) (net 18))
 (segment (start 151.003 100.965) (end 151.638 100.33) (width 0.3) (layer F.Cu) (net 18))
 (segment (start 151.638 100.33) (end 151.638 93.345) (width 0.3) (layer F.Cu) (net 18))
 (segment (start 136.578 99.441) (end 139.192 99.441) (width 0.6) (layer F.Cu) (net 11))
 (segment (start 139.446 99.695) (end 139.446 100.277) (width 0.6) (layer F.Cu) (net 11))
 (segment (start 139.192 99.441) (end 139.446 99.695) (width 0.6) (layer F.Cu) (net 11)))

